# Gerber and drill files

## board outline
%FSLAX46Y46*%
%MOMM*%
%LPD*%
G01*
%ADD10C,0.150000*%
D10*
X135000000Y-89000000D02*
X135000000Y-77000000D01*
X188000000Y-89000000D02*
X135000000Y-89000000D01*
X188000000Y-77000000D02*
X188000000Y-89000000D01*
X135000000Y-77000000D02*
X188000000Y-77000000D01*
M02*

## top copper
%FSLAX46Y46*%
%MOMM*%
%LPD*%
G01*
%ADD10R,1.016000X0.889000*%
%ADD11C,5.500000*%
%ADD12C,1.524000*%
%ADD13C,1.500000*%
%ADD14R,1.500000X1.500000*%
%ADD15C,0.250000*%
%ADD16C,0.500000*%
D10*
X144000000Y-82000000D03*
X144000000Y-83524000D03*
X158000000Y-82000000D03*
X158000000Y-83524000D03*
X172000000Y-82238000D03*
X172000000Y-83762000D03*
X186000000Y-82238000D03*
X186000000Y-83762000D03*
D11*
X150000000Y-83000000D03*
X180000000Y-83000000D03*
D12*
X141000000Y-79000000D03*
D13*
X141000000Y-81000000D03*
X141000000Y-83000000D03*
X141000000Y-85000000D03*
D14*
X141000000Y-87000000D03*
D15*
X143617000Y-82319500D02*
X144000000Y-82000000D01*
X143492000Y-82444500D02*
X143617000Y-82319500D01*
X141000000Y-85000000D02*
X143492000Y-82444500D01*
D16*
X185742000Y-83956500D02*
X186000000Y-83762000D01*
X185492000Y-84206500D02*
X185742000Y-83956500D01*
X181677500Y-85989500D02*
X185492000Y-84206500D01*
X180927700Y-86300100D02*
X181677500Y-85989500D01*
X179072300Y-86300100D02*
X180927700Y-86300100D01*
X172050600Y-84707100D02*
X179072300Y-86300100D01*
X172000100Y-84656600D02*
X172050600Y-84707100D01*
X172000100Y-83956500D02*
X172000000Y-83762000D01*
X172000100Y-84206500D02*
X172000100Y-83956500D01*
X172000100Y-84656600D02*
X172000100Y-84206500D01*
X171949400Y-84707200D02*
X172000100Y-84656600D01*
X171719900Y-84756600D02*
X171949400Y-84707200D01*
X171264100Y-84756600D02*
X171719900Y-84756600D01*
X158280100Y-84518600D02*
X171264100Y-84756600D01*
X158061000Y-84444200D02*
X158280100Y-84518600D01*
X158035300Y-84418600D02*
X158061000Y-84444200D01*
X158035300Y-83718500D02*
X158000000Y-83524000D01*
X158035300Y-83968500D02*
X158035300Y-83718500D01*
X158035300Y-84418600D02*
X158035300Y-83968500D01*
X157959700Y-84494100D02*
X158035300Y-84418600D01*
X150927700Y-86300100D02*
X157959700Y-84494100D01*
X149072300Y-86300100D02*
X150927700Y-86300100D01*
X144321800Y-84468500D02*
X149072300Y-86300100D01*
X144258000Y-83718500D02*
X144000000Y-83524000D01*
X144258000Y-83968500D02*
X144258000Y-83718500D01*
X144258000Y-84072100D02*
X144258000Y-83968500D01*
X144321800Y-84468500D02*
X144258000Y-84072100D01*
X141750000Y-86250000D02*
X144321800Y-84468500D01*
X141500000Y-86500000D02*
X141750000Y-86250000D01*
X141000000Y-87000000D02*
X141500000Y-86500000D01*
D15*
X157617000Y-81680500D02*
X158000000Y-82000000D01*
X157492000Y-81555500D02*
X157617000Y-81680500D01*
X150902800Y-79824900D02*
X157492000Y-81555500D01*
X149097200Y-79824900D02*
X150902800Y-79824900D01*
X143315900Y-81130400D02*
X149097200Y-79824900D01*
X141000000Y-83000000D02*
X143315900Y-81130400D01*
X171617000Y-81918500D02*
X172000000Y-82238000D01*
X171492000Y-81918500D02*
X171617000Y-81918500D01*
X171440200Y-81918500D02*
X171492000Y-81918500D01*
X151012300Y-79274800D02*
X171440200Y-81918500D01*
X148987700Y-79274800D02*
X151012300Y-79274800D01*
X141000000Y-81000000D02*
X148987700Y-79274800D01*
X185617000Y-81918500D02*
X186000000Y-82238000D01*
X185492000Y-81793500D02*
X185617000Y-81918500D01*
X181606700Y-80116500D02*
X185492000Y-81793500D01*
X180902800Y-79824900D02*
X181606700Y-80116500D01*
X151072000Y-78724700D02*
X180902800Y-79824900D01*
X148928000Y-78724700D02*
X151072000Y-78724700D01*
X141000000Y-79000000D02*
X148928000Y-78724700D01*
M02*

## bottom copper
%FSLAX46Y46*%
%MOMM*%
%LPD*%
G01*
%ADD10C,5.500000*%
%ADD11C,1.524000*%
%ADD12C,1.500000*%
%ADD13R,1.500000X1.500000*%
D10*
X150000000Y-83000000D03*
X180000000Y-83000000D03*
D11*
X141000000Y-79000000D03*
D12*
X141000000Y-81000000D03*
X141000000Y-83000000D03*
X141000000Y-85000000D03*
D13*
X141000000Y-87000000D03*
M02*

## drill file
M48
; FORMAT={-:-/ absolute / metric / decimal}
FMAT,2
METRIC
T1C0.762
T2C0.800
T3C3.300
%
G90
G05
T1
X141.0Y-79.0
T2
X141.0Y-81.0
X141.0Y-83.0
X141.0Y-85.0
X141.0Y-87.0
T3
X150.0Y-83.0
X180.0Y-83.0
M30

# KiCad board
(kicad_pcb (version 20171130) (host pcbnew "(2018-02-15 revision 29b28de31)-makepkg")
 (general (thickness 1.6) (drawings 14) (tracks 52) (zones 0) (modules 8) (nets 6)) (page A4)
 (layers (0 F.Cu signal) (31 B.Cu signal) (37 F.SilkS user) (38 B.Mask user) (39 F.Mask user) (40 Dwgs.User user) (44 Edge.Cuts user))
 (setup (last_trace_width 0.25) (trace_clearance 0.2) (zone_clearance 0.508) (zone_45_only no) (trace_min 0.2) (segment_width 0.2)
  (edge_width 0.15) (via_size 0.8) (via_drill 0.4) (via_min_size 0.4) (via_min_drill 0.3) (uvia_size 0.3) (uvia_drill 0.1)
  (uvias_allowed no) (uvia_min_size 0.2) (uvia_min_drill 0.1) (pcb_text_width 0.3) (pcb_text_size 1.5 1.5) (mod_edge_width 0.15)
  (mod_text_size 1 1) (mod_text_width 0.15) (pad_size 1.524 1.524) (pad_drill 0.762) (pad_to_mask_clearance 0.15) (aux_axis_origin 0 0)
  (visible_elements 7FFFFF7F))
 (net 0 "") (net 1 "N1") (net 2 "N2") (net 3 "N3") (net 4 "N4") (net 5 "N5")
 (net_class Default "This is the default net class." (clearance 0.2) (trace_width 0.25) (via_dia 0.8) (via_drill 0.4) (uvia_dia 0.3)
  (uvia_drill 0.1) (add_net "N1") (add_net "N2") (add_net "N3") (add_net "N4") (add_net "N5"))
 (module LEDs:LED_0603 (layer F.Cu) (at 144 82.762 270)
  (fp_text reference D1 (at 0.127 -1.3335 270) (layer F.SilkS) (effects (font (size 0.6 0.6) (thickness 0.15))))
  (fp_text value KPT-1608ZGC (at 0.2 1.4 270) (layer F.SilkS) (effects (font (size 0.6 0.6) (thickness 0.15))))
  (pad A smd rect (at -0.762 0 270) (size 0.889 1.016) (layers F.Cu F.Mask) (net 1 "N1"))
  (pad C smd rect (at 0.762 0 270) (size 0.889 1.016) (layers F.Cu F.Mask) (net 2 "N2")))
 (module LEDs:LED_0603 (layer F.Cu) (at 158 82.762 270)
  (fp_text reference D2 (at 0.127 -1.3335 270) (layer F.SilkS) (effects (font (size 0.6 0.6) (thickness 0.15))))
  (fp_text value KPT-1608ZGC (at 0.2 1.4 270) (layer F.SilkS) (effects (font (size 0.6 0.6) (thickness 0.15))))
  (pad A smd rect (at -0.762 0 270) (size 0.889 1.016) (layers F.Cu F.Mask) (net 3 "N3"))
  (pad C smd rect (at 0.762 0 270) (size 0.889 1.016) (layers F.Cu F.Mask) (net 2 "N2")))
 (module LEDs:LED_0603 (layer F.Cu) (at 172 83 270)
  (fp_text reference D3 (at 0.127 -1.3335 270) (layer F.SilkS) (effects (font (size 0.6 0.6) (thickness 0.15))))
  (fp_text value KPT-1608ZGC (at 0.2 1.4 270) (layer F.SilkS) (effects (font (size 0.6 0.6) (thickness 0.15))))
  (pad A smd rect (at -0.762 0 270) (size 0.889 1.016) (layers F.Cu F.Mask) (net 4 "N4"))
  (pad C smd rect (at 0.762 0 270) (size 0.889 1.016) (layers F.Cu F.Mask) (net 2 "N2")))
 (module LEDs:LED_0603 (layer F.Cu) (at 186 83 270)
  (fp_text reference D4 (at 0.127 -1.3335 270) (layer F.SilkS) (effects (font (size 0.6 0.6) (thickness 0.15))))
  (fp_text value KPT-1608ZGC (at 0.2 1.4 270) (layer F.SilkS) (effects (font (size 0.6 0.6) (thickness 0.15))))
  (pad A smd rect (at -0.762 0 270) (size 0.889 1.016) (layers F.Cu F.Mask) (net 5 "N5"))
  (pad C smd rect (at 0.762 0 270) (size 0.889 1.016) (layers F.Cu F.Mask) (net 2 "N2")))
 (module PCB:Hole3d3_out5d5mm (layer F.Cu) (at 150 83)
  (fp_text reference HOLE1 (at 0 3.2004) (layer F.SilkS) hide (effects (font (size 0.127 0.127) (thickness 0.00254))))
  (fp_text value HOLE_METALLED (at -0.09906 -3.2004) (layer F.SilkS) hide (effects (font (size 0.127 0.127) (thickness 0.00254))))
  (pad H thru_hole circle (at 0 0) (size 5.5 5.5) (drill 3.3) (layers *.Cu *.Mask F.SilkS)))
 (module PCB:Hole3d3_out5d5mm (layer F.Cu) (at 180 83)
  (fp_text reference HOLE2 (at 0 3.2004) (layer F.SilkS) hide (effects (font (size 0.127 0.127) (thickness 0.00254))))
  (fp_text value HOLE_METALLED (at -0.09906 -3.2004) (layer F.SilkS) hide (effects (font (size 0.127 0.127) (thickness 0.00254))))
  (pad H thru_hole circle (at 0 0) (size 5.5 5.5) (drill 3.3) (layers *.Cu *.Mask F.SilkS)))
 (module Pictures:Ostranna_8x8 (layer F.Cu) (at 165 83)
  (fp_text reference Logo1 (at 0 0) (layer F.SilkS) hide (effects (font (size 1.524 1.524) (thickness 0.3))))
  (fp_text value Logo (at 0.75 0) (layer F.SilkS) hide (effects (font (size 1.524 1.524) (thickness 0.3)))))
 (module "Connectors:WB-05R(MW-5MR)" (layer F.Cu) (at 141 83 90)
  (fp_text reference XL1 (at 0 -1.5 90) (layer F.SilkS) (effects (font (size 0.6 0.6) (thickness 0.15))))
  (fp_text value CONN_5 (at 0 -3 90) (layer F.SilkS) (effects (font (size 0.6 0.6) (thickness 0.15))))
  (pad 5 thru_hole circle (at 4 0 90) (size 1.524 1.524) (drill 0.762) (layers *.Cu *.Mask) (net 5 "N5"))
  (pad 4 thru_hole circle (at 2 0 90) (size 1.5 1.5) (drill 0.8) (layers *.Cu *.Mask F.SilkS) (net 4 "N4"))
  (pad 3 thru_hole circle (at 0 0 90) (size 1.5 1.5) (drill 0.8) (layers *.Cu *.Mask F.SilkS) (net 3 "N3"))
  (pad 2 thru_hole circle (at -2 0 90) (size 1.5 1.5) (drill 0.8) (layers *.Cu *.Mask F.SilkS) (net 1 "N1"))
  (pad 1 thru_hole rect (at -4 0 90) (size 1.5 1.5) (drill 0.8) (layers *.Cu *.Mask F.SilkS) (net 2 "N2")))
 (gr_line (start 135 89) (end 135 77) (layer Edge.Cuts) (width 0.15))
 (gr_line (start 188 89) (end 135 89) (layer Edge.Cuts) (width 0.15))
 (gr_line (start 188 77) (end 188 89) (layer Edge.Cuts) (width 0.15))
 (gr_line (start 135 77) (end 188 77) (layer Edge.Cuts) (width 0.15))
 (segment (start 143.617 82.3195) (end 144 82) (width 0.25) (layer F.Cu) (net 1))
 (segment (start 143.492 82.4445) (end 143.617 82.3195) (width 0.25) (layer F.Cu) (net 1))
 (segment (start 141 85) (end 143.492 82.4445) (width 0.25) (layer F.Cu) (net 1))
 (segment (start 185.742 83.9565) (end 186 83.762) (width 0.5) (layer F.Cu) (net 2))
 (segment (start 185.492 84.2065) (end 185.742 83.9565) (width 0.5) (layer F.Cu) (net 2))
 (segment (start 181.6775 85.9895) (end 185.492 84.2065) (width 0.5) (layer F.Cu) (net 2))
 (segment (start 180.9277 86.3001) (end 181.6775 85.9895) (width 0.5) (layer F.Cu) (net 2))
 (segment (start 179.0723 86.3001) (end 180.9277 86.3001) (width 0.5) (layer F.Cu) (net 2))
 (segment (start 172.0506 84.7071) (end 179.0723 86.3001) (width 0.5) (layer F.Cu) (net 2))
 (segment (start 172.0001 84.6566) (end 172.0506 84.7071) (width 0.5) (layer F.Cu) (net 2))
 (segment (start 172.0001 83.9565) (end 172 83.762) (width 0.5) (layer F.Cu) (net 2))
 (segment (start 172.0001 84.2065) (end 172.0001 83.9565) (width 0.5) (layer F.Cu) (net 2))
 (segment (start 172.0001 84.6566) (end 172.0001 84.2065) (width 0.5) (layer F.Cu) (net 2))
 (segment (start 171.9494 84.7072) (end 172.0001 84.6566) (width 0.5) (layer F.Cu) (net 2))
 (segment (start 171.7199 84.7566) (end 171.9494 84.7072) (width 0.5) (layer F.Cu) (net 2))
 (segment (start 171.2641 84.7566) (end 171.7199 84.7566) (width 0.5) (layer F.Cu) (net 2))
 (segment (start 158.2801 84.5186) (end 171.2641 84.7566) (width 0.5) (layer F.Cu) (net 2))
 (segment (start 158.061 84.4442) (end 158.2801 84.5186) (width 0.5) (layer F.Cu) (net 2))
 (segment (start 158.0353 84.4186) (end 158.061 84.4442) (width 0.5) (layer F.Cu) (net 2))
 (segment (start 158.0353 83.7185) (end 158 83.524) (width 0.5) (layer F.Cu) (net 2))
 (segment (start 158.0353 83.9685) (end 158.0353 83.7185) (width 0.5) (layer F.Cu) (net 2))
 (segment (start 158.0353 84.4186) (end 158.0353 83.9685) (width 0.5) (layer F.Cu) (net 2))
 (segment (start 157.9597 84.4941) (end 158.0353 84.4186) (width 0.5) (layer F.Cu) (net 2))
 (segment (start 150.9277 86.3001) (end 157.9597 84.4941) (width 0.5) (layer F.Cu) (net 2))
 (segment (start 149.0723 86.3001) (end 150.9277 86.3001) (width 0.5) (layer F.Cu) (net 2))
 (segment (start 144.3218 84.4685) (end 149.0723 86.3001) (width 0.5) (layer F.Cu) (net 2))
 (segment (start 144.258 83.7185) (end 144 83.524) (width 0.5) (layer F.Cu) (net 2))
 (segment (start 144.258 83.9685) (end 144.258 83.7185) (width 0.5) (layer F.Cu) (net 2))
 (segment (start 144.258 84.0721) (end 144.258 83.9685) (width 0.5) (layer F.Cu) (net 2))
 (segment (start 144.3218 84.4685) (end 144.258 84.0721) (width 0.5) (layer F.Cu) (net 2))
 (segment (start 141.75 86.25) (end 144.3218 84.4685) (width 0.5) (layer F.Cu) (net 2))
 (segment (start 141.5 86.5) (end 141.75 86.25) (width 0.5) (layer F.Cu) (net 2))
 (segment (start 141 87) (end 141.5 86.5) (width 0.5) (layer F.Cu) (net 2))
 (segment (start 157.617 81.6805) (end 158 82) (width 0.25) (layer F.Cu) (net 3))
 (segment (start 157.492 81.5555) (end 157.617 81.6805) (width 0.25) (layer F.Cu) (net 3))
 (segment (start 150.9028 79.8249) (end 157.492 81.5555) (width 0.25) (layer F.Cu) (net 3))
 (segment (start 149.0972 79.8249) (end 150.9028 79.8249) (width 0.25) (layer F.Cu) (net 3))
 (segment (start 143.3159 81.1304) (end 149.0972 79.8249) (width 0.25) (layer F.Cu) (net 3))
 (segment (start 141 83) (end 143.3159 81.1304) (width 0.25) (layer F.Cu) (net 3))
 (segment (start 171.617 81.9185) (end 172 82.238) (width 0.25) (layer F.Cu) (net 4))
 (segment (start 171.492 81.9185) (end 171.617 81.9185) (width 0.25) (layer F.Cu) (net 4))
 (segment (start 171.4402 81.9185) (end 171.492 81.9185) (width 0.25) (layer F.Cu) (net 4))
 (segment (start 151.0123 79.2748) (end 171.4402 81.9185) (width 0.25) (layer F.Cu) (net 4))
 (segment (start 148.9877 79.2748) (end 151.0123 79.2748) (width 0.25) (layer F.Cu) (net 4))
 (segment (start 141 81) (end 148.9877 79.2748) (width 0.25) (layer F.Cu) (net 4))
 (segment (start 185.617 81.9185) (end 186 82.238) (width 0.25) (layer F.Cu) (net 5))
 (segment (start 185.492 81.7935) (end 185.617 81.9185) (width 0.25) (layer F.Cu) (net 5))
 (segment (start 181.6067 80.1165) (end 185.492 81.7935) (width 0.25) (layer F.Cu) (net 5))
 (segment (start 180.9028 79.8249) (end 181.6067 80.1165) (width 0.25) (layer F.Cu) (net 5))
 (segment (start 151.072 78.7247) (end 180.9028 79.8249) (width 0.25) (layer F.Cu) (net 5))
 (segment (start 148.928 78.7247) (end 151.072 78.7247) (width 0.25) (layer F.Cu) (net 5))
 (segment (start 141 79) (end 148.928 78.7247) (width 0.25) (layer F.Cu) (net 5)))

